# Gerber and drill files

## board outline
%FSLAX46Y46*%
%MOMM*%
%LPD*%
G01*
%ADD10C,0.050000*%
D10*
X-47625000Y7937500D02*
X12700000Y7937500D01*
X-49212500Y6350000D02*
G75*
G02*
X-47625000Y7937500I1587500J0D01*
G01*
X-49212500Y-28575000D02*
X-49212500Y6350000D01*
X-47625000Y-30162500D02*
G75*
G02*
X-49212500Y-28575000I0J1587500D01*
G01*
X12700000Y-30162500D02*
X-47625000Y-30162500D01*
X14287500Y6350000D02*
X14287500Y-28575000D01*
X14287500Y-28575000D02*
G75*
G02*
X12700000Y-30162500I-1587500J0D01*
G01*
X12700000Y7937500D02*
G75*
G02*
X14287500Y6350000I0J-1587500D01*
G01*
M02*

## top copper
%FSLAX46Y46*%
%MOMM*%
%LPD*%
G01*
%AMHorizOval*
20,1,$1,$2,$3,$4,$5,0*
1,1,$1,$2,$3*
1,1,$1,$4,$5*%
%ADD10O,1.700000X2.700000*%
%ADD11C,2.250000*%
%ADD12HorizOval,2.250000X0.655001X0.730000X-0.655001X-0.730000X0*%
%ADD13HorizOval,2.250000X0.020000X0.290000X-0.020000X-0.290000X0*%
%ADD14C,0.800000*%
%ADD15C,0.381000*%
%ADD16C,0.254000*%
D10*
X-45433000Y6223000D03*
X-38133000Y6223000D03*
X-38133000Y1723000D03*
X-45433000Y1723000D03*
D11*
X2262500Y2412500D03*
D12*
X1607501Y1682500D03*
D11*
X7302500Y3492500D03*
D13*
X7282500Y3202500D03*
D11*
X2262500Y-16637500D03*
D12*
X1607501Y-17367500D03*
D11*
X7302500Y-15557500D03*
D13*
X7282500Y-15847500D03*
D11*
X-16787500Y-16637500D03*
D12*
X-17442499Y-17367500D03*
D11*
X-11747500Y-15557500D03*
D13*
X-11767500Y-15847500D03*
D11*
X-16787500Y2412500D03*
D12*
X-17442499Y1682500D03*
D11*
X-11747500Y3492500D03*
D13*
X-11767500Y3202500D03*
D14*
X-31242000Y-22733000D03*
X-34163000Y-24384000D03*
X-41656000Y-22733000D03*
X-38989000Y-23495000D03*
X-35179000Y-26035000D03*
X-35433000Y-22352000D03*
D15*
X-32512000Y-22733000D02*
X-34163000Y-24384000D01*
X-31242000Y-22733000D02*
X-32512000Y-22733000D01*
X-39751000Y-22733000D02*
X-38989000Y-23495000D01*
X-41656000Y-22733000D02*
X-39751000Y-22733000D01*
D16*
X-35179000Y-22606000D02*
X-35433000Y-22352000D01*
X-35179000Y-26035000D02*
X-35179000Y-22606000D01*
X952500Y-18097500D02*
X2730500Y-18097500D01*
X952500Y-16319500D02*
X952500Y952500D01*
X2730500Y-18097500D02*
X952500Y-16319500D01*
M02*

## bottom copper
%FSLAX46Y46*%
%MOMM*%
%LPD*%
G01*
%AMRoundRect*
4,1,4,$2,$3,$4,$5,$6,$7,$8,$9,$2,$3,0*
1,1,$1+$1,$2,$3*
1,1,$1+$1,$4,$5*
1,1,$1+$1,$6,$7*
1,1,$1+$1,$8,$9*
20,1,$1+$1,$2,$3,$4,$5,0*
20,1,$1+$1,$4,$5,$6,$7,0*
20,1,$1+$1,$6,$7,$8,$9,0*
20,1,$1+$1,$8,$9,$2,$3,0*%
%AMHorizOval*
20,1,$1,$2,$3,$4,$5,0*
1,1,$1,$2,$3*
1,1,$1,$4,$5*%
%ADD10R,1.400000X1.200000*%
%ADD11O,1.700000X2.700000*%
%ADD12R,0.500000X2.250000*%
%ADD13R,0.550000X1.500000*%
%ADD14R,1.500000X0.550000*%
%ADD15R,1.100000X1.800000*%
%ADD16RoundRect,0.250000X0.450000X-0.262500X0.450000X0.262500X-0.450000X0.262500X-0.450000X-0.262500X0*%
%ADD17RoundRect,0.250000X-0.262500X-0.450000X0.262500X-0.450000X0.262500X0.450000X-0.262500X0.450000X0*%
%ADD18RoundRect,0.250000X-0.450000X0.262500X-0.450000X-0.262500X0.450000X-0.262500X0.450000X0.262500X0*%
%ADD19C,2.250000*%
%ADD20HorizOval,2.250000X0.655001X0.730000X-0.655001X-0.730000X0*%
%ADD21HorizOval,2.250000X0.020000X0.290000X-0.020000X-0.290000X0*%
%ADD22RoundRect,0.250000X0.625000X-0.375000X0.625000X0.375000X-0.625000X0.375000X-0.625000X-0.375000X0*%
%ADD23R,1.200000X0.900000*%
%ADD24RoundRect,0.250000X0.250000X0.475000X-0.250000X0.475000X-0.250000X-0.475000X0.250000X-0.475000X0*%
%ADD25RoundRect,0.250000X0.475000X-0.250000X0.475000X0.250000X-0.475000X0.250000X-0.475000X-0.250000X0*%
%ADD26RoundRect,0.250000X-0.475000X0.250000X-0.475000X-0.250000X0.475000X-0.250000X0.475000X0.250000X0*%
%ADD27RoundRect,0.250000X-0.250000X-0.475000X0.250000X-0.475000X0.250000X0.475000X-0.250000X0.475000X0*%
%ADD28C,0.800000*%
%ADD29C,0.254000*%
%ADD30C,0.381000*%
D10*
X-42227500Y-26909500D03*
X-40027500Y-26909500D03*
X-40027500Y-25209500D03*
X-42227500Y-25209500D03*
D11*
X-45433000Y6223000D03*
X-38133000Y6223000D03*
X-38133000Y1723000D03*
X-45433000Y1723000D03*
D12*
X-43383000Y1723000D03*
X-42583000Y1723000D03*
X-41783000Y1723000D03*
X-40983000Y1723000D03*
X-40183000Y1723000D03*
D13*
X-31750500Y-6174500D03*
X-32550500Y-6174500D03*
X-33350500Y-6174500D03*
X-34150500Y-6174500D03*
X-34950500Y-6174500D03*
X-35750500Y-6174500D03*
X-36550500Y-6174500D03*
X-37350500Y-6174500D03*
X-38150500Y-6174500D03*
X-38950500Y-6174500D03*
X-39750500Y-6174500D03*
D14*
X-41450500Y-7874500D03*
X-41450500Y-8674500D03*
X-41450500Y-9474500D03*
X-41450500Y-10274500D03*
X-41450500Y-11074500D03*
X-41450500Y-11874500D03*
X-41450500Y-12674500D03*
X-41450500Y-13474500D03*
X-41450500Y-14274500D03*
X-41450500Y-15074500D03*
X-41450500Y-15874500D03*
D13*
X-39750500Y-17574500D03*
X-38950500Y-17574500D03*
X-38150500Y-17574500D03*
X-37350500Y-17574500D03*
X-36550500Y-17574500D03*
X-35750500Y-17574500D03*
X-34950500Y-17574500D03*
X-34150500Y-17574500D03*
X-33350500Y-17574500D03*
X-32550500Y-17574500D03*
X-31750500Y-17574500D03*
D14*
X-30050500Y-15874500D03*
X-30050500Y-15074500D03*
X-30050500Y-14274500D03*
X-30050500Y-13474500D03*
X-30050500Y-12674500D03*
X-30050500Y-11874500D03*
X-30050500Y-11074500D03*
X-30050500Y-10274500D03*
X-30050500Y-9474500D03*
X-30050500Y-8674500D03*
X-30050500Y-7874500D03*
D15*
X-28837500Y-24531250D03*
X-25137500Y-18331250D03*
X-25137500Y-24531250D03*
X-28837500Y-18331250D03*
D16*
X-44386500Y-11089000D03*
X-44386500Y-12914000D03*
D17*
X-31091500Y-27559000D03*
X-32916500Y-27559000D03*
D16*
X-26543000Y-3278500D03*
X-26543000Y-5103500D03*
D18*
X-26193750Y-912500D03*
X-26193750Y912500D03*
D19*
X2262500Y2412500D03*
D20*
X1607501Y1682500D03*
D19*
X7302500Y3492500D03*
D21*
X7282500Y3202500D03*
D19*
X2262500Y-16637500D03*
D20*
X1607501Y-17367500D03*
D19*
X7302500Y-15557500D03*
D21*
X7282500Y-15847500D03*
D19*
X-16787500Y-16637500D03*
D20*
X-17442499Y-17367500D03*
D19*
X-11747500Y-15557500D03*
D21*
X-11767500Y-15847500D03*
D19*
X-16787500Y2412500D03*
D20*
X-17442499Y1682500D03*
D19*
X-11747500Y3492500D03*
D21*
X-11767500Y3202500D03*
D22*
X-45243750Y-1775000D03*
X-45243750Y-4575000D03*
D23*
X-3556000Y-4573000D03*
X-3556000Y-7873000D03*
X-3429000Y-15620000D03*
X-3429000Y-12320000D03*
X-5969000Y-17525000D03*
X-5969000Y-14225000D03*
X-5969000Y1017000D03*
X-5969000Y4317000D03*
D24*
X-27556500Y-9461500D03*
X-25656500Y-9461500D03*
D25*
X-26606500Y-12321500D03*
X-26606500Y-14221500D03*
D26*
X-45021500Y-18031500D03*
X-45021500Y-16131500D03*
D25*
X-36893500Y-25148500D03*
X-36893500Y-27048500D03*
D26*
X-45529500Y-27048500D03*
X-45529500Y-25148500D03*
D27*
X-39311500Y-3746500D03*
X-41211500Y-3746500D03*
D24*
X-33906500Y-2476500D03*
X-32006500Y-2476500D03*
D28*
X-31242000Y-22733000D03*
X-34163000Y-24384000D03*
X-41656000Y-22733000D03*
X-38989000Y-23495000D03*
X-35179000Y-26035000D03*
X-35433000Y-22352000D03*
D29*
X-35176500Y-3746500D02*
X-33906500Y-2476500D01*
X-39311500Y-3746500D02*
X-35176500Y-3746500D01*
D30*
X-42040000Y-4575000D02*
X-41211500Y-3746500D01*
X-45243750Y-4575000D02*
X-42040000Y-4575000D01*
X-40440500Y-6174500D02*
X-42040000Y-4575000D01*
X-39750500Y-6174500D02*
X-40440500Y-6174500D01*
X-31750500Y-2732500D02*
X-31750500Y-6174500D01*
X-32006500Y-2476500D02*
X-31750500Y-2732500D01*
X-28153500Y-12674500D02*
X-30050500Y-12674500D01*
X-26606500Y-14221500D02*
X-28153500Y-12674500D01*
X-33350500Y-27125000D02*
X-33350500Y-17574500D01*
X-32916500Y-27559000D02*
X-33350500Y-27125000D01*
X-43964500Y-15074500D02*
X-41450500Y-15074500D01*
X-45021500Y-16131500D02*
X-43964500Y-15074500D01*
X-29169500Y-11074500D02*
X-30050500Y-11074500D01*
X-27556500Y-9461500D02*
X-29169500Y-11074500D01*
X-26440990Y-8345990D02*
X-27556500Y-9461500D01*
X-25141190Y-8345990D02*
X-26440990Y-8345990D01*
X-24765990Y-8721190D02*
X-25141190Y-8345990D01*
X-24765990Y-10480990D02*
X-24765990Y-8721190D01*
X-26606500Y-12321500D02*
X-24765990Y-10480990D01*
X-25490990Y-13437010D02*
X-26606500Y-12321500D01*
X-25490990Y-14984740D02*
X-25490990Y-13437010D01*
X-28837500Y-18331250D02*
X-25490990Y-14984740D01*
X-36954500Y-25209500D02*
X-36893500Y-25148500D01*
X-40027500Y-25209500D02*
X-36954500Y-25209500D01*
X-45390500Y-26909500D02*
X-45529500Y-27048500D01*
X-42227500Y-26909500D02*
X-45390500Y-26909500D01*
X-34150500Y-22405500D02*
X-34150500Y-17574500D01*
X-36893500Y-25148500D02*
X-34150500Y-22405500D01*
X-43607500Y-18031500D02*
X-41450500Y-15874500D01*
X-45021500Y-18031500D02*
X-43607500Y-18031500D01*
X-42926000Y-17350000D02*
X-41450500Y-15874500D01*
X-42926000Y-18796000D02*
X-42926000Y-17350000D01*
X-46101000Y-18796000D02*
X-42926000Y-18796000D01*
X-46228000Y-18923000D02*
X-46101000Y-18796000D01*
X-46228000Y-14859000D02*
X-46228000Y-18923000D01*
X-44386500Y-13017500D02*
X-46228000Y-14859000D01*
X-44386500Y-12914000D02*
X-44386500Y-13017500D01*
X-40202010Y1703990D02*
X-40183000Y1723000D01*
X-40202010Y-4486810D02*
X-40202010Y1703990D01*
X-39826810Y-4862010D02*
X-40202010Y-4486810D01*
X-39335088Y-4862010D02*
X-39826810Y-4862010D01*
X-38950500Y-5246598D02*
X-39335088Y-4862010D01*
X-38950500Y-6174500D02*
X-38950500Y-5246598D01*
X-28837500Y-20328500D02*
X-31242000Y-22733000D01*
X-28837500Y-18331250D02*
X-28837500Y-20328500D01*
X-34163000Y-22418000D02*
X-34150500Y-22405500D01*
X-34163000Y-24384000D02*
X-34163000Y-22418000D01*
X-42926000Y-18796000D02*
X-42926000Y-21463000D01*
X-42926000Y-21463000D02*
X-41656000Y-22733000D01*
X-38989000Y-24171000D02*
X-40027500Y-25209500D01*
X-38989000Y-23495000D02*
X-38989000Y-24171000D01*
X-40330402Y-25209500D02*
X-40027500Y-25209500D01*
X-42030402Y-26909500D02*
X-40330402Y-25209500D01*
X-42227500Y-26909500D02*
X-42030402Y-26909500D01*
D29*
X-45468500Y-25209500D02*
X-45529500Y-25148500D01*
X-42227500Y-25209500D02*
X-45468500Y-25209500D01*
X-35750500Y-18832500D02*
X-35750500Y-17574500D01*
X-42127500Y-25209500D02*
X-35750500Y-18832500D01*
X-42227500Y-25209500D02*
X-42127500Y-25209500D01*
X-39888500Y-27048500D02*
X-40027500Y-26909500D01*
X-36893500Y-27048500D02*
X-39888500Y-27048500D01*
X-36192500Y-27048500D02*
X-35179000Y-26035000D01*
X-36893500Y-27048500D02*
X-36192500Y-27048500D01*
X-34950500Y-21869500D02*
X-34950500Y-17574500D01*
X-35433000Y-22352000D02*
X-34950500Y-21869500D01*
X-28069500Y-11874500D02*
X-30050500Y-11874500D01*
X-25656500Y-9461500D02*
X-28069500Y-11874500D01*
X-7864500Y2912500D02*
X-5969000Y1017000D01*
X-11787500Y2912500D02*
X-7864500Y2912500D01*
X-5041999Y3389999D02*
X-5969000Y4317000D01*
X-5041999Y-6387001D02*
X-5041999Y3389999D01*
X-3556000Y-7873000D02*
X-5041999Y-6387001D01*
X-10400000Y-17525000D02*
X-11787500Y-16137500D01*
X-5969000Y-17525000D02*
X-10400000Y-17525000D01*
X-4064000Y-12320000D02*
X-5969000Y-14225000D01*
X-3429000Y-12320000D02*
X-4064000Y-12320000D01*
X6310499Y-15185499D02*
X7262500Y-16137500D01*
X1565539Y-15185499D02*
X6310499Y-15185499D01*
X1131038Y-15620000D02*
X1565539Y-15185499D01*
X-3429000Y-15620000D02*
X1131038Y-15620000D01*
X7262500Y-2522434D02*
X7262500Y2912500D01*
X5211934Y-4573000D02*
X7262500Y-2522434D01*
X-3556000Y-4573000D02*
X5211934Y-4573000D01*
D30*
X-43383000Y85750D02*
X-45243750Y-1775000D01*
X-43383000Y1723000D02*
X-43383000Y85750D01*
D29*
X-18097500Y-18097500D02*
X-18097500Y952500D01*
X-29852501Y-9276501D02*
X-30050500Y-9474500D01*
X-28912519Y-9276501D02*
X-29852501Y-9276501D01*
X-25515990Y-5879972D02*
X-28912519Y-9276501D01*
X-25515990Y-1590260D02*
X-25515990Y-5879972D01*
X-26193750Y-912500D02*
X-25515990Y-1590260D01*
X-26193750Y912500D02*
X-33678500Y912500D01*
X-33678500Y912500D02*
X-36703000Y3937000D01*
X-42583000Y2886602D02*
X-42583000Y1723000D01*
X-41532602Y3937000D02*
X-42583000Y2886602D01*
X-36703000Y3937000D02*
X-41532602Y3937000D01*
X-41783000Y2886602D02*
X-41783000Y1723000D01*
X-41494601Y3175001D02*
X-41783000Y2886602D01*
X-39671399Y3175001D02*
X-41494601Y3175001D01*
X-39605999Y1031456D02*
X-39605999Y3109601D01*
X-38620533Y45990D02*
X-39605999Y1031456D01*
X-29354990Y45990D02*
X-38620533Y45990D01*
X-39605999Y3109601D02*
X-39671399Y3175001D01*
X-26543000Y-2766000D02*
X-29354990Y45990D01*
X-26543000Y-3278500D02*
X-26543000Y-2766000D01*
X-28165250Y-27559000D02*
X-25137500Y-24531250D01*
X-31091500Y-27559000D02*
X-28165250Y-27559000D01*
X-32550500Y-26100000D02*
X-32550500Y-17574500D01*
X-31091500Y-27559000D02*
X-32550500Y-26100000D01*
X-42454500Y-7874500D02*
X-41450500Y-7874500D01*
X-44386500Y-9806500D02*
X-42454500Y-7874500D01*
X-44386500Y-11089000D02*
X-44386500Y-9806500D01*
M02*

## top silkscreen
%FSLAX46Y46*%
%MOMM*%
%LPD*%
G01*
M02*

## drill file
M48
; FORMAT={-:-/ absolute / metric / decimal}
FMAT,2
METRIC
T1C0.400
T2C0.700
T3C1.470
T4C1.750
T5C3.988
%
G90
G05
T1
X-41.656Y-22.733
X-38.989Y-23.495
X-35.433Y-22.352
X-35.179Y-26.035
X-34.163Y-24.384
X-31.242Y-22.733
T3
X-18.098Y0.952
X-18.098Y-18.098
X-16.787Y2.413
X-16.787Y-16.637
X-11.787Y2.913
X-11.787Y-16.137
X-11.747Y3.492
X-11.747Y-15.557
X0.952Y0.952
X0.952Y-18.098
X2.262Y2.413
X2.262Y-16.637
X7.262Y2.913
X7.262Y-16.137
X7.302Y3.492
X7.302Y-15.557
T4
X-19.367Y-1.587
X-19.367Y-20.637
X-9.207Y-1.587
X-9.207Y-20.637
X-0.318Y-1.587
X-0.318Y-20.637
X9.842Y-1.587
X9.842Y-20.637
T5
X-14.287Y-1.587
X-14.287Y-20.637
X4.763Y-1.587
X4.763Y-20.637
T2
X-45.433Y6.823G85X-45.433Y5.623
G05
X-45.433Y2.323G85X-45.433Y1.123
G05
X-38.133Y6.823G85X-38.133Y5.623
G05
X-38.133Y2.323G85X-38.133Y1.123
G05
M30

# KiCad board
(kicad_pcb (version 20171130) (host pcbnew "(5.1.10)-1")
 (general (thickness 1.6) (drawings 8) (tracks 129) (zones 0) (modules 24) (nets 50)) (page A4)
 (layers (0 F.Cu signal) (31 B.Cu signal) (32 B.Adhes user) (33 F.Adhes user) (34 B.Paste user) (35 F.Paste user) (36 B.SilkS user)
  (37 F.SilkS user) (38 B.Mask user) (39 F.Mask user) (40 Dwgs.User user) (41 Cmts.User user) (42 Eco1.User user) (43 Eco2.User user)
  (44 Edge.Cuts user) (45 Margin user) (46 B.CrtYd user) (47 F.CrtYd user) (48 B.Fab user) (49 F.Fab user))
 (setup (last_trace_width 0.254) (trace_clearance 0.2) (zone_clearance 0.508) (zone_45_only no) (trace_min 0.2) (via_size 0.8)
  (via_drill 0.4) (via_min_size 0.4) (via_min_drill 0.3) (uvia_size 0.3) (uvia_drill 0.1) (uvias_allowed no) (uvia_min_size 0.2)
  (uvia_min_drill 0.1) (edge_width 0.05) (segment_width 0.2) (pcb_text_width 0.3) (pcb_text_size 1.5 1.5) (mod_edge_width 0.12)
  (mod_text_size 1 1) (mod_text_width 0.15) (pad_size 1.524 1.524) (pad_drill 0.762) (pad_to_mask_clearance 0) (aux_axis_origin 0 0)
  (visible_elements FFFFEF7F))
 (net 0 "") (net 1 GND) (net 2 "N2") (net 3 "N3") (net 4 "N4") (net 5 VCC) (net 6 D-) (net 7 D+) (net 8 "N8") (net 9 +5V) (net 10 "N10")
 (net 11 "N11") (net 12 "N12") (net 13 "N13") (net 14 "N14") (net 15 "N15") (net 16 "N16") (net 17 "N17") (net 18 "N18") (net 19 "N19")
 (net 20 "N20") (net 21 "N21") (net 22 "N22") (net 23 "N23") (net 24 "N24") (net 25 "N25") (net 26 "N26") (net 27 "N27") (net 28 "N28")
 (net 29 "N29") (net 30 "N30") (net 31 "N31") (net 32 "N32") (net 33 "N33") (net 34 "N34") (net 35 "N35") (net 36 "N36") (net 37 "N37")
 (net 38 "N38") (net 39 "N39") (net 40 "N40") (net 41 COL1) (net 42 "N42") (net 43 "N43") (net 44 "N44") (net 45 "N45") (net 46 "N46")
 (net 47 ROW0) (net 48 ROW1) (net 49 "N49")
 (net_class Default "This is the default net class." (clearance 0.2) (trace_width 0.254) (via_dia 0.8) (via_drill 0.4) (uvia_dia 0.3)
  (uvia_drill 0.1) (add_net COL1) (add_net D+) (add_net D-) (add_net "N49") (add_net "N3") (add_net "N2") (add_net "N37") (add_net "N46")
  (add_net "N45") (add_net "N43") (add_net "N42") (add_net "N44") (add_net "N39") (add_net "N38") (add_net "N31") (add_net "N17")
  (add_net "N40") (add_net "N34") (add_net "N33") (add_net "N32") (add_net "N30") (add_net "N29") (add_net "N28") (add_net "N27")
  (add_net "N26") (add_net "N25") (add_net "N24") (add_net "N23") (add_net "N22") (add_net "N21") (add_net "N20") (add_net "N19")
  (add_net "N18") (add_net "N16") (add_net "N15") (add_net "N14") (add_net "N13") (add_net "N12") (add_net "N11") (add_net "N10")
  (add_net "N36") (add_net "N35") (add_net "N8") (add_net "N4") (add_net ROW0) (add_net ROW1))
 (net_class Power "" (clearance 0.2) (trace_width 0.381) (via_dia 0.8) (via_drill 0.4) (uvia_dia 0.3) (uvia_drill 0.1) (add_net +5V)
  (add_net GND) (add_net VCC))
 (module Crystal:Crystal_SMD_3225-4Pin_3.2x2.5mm (layer B.Cu) (at -41.1275 26.0595)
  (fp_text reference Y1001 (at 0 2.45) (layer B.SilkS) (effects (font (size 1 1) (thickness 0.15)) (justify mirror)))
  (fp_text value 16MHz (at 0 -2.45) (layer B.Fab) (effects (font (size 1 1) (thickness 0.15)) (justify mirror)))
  (pad 4 smd rect (at -1.1 0.85) (size 1.4 1.2) (layers B.Cu B.Paste B.Mask) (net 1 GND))
  (pad 3 smd rect (at 1.1 0.85) (size 1.4 1.2) (layers B.Cu B.Paste B.Mask) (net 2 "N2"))
  (pad 2 smd rect (at 1.1 -0.85) (size 1.4 1.2) (layers B.Cu B.Paste B.Mask) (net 1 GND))
  (pad 1 smd rect (at -1.1 -0.85) (size 1.4 1.2) (layers B.Cu B.Paste B.Mask) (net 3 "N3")))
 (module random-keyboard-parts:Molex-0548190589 (layer B.Cu) (at -41.783 -6.223 270)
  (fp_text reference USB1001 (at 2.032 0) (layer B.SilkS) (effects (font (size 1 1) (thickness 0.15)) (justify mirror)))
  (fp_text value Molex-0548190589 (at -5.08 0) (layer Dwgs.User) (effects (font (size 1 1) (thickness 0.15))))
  (pad 6 thru_hole oval (at 0 3.65 270) (size 2.7 1.7) (drill oval 1.9 0.7) (layers *.Cu *.Mask) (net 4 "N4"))
  (pad 6 thru_hole oval (at 0 -3.65 270) (size 2.7 1.7) (drill oval 1.9 0.7) (layers *.Cu *.Mask) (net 4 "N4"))
  (pad 6 thru_hole oval (at 4.5 -3.65 270) (size 2.7 1.7) (drill oval 1.9 0.7) (layers *.Cu *.Mask) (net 4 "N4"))
  (pad 6 thru_hole oval (at 4.5 3.65 270) (size 2.7 1.7) (drill oval 1.9 0.7) (layers *.Cu *.Mask) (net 4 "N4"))
  (pad 5 smd rect (at 4.5 1.6 270) (size 2.25 0.5) (layers B.Cu B.Paste B.Mask) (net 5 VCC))
  (pad 4 smd rect (at 4.5 0.8 270) (size 2.25 0.5) (layers B.Cu B.Paste B.Mask) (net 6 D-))
  (pad 3 smd rect (at 4.5 0 270) (size 2.25 0.5) (layers B.Cu B.Paste B.Mask) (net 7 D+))
  (pad 2 smd rect (at 4.5 -0.8 270) (size 2.25 0.5) (layers B.Cu B.Paste B.Mask) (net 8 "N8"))
  (pad 1 smd rect (at 4.5 -1.6 270) (size 2.25 0.5) (layers B.Cu B.Paste B.Mask) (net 1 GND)))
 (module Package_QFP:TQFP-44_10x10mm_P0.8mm (layer B.Cu) (at -35.7505 11.8745 180)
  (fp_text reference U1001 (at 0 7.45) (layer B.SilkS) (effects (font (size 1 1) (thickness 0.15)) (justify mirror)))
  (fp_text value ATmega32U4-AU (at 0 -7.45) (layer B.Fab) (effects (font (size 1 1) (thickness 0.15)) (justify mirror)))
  (pad 44 smd rect (at -4 5.7 90) (size 1.5 0.55) (layers B.Cu B.Paste B.Mask) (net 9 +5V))
  (pad 43 smd rect (at -3.2 5.7 90) (size 1.5 0.55) (layers B.Cu B.Paste B.Mask) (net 1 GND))
  (pad 42 smd rect (at -2.4 5.7 90) (size 1.5 0.55) (layers B.Cu B.Paste B.Mask) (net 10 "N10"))
  (pad 41 smd rect (at -1.6 5.7 90) (size 1.5 0.55) (layers B.Cu B.Paste B.Mask) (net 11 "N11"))
  (pad 40 smd rect (at -0.8 5.7 90) (size 1.5 0.55) (layers B.Cu B.Paste B.Mask) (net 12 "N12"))
  (pad 39 smd rect (at 0 5.7 90) (size 1.5 0.55) (layers B.Cu B.Paste B.Mask) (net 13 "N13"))
  (pad 38 smd rect (at 0.8 5.7 90) (size 1.5 0.55) (layers B.Cu B.Paste B.Mask) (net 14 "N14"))
  (pad 37 smd rect (at 1.6 5.7 90) (size 1.5 0.55) (layers B.Cu B.Paste B.Mask) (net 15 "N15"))
  (pad 36 smd rect (at 2.4 5.7 90) (size 1.5 0.55) (layers B.Cu B.Paste B.Mask) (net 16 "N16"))
  (pad 35 smd rect (at 3.2 5.7 90) (size 1.5 0.55) (layers B.Cu B.Paste B.Mask) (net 1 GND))
  (pad 34 smd rect (at 4 5.7 90) (size 1.5 0.55) (layers B.Cu B.Paste B.Mask) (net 9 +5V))
  (pad 33 smd rect (at 5.7 4 180) (size 1.5 0.55) (layers B.Cu B.Paste B.Mask) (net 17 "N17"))
  (pad 32 smd rect (at 5.7 3.2 180) (size 1.5 0.55) (layers B.Cu B.Paste B.Mask) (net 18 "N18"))
  (pad 31 smd rect (at 5.7 2.4 180) (size 1.5 0.55) (layers B.Cu B.Paste B.Mask) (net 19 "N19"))
  (pad 30 smd rect (at 5.7 1.6 180) (size 1.5 0.55) (layers B.Cu B.Paste B.Mask) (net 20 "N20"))
  (pad 29 smd rect (at 5.7 0.8 180) (size 1.5 0.55) (layers B.Cu B.Paste B.Mask) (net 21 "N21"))
  (pad 28 smd rect (at 5.7 0 180) (size 1.5 0.55) (layers B.Cu B.Paste B.Mask) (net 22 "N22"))
  (pad 27 smd rect (at 5.7 -0.8 180) (size 1.5 0.55) (layers B.Cu B.Paste B.Mask) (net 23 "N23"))
  (pad 26 smd rect (at 5.7 -1.6 180) (size 1.5 0.55) (layers B.Cu B.Paste B.Mask) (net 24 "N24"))
  (pad 25 smd rect (at 5.7 -2.4 180) (size 1.5 0.55) (layers B.Cu B.Paste B.Mask) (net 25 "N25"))
  (pad 24 smd rect (at 5.7 -3.2 180) (size 1.5 0.55) (layers B.Cu B.Paste B.Mask) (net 9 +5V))
  (pad 23 smd rect (at 5.7 -4 180) (size 1.5 0.55) (layers B.Cu B.Paste B.Mask) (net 1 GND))
  (pad 22 smd rect (at 4 -5.7 90) (size 1.5 0.55) (layers B.Cu B.Paste B.Mask) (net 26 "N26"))
  (pad 21 smd rect (at 3.2 -5.7 90) (size 1.5 0.55) (layers B.Cu B.Paste B.Mask) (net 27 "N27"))
  (pad 20 smd rect (at 2.4 -5.7 90) (size 1.5 0.55) (layers B.Cu B.Paste B.Mask) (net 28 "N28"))
  (pad 19 smd rect (at 1.6 -5.7 90) (size 1.5 0.55) (layers B.Cu B.Paste B.Mask) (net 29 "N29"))
  (pad 18 smd rect (at 0.8 -5.7 90) (size 1.5 0.55) (layers B.Cu B.Paste B.Mask) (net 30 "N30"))
  (pad 17 smd rect (at 0 -5.7 90) (size 1.5 0.55) (layers B.Cu B.Paste B.Mask) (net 3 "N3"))
  (pad 16 smd rect (at -0.8 -5.7 90) (size 1.5 0.55) (layers B.Cu B.Paste B.Mask) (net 2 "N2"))
  (pad 15 smd rect (at -1.6 -5.7 90) (size 1.5 0.55) (layers B.Cu B.Paste B.Mask) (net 1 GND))
  (pad 14 smd rect (at -2.4 -5.7 90) (size 1.5 0.55) (layers B.Cu B.Paste B.Mask) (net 9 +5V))
  (pad 13 smd rect (at -3.2 -5.7 90) (size 1.5 0.55) (layers B.Cu B.Paste B.Mask) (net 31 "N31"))
  (pad 12 smd rect (at -4 -5.7 90) (size 1.5 0.55) (layers B.Cu B.Paste B.Mask) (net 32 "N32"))
  (pad 11 smd rect (at -5.7 -4 180) (size 1.5 0.55) (layers B.Cu B.Paste B.Mask) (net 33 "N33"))
  (pad 10 smd rect (at -5.7 -3.2 180) (size 1.5 0.55) (layers B.Cu B.Paste B.Mask) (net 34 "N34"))
  (pad 9 smd rect (at -5.7 -2.4 180) (size 1.5 0.55) (layers B.Cu B.Paste B.Mask) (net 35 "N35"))
  (pad 8 smd rect (at -5.7 -1.6 180) (size 1.5 0.55) (layers B.Cu B.Paste B.Mask) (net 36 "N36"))
  (pad 7 smd rect (at -5.7 -0.8 180) (size 1.5 0.55) (layers B.Cu B.Paste B.Mask) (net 9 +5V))
  (pad 6 smd rect (at -5.7 0 180) (size 1.5 0.55) (layers B.Cu B.Paste B.Mask) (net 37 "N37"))
  (pad 5 smd rect (at -5.7 0.8 180) (size 1.5 0.55) (layers B.Cu B.Paste B.Mask) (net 1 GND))
  (pad 4 smd rect (at -5.7 1.6 180) (size 1.5 0.55) (layers B.Cu B.Paste B.Mask) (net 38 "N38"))
  (pad 3 smd rect (at -5.7 2.4 180) (size 1.5 0.55) (layers B.Cu B.Paste B.Mask) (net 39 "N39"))
  (pad 2 smd rect (at -5.7 3.2 180) (size 1.5 0.55) (layers B.Cu B.Paste B.Mask) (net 9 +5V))
  (pad 1 smd rect (at -5.7 4 180) (size 1.5 0.55) (layers B.Cu B.Paste B.Mask) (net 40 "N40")))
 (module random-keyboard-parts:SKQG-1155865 (layer B.Cu) (at -26.9875 21.43125 90)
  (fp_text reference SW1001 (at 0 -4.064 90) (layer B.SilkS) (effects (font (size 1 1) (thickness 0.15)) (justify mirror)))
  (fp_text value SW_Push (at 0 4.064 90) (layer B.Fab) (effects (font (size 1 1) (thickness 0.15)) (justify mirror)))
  (pad 4 smd rect (at -3.1 -1.85 90) (size 1.8 1.1) (layers B.Cu B.Paste B.Mask))
  (pad 3 smd rect (at 3.1 1.85 90) (size 1.8 1.1) (layers B.Cu B.Paste B.Mask))
  (pad 2 smd rect (at -3.1 1.85 90) (size 1.8 1.1) (layers B.Cu B.Paste B.Mask) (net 31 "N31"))
  (pad 1 smd rect (at 3.1 -1.85 90) (size 1.8 1.1) (layers B.Cu B.Paste B.Mask) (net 1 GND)))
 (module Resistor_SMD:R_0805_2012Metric (layer B.Cu) (at -44.3865 12.0015 90)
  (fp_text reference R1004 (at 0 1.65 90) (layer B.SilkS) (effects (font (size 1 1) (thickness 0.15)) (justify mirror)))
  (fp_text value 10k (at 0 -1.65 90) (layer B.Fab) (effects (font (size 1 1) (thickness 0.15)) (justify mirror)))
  (pad 2 smd roundrect (at 0.9125 0 90) (size 1.025 1.4) (layers B.Cu B.Paste B.Mask) (roundrect_rratio 0.243902) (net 17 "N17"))
  (pad 1 smd roundrect (at -0.9125 0 90) (size 1.025 1.4) (layers B.Cu B.Paste B.Mask) (roundrect_rratio 0.243902) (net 1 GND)))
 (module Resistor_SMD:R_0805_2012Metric (layer B.Cu) (at -32.004 27.559)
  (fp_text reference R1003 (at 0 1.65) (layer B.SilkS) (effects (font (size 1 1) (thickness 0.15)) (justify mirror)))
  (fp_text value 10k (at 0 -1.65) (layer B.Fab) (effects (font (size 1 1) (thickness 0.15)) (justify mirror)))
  (pad 2 smd roundrect (at 0.9125 0) (size 1.025 1.4) (layers B.Cu B.Paste B.Mask) (roundrect_rratio 0.243902) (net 31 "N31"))
  (pad 1 smd roundrect (at -0.9125 0) (size 1.025 1.4) (layers B.Cu B.Paste B.Mask) (roundrect_rratio 0.243902) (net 9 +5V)))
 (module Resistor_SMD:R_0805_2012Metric (layer B.Cu) (at -26.543 4.191 90)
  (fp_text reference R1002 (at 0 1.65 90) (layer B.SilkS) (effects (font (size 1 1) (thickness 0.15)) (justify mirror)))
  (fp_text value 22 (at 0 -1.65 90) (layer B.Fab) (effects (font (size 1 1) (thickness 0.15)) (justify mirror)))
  (pad 2 smd roundrect (at 0.9125 0 90) (size 1.025 1.4) (layers B.Cu B.Paste B.Mask) (roundrect_rratio 0.243902) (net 7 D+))
  (pad 1 smd roundrect (at -0.9125 0 90) (size 1.025 1.4) (layers B.Cu B.Paste B.Mask) (roundrect_rratio 0.243902) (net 38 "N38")))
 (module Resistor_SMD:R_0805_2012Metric (layer B.Cu) (at -26.19375 0 270)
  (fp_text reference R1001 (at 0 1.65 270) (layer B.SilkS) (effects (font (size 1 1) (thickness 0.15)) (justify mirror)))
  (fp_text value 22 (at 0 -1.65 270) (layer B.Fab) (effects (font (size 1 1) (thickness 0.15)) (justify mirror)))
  (pad 2 smd roundrect (at 0.9125 0 270) (size 1.025 1.4) (layers B.Cu B.Paste B.Mask) (roundrect_rratio 0.243902) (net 39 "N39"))
  (pad 1 smd roundrect (at -0.9125 0 270) (size 1.025 1.4) (layers B.Cu B.Paste B.Mask) (roundrect_rratio 0.243902) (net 6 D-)))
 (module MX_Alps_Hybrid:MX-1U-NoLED (layer F.Cu) (at 4.7625 1.5875)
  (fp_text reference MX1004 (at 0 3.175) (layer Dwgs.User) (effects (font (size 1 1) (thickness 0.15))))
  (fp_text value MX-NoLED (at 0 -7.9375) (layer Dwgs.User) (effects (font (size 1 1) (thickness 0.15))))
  (pad "" np_thru_hole circle (at 5.08 0 48.0996) (size 1.75 1.75) (drill 1.75) (layers *.Cu *.Mask))
  (pad "" np_thru_hole circle (at -5.08 0 48.0996) (size 1.75 1.75) (drill 1.75) (layers *.Cu *.Mask))
  (pad 1 thru_hole circle (at -2.5 -4) (size 2.25 2.25) (drill 1.47) (layers *.Cu B.Mask) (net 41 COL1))
  (pad "" np_thru_hole circle (at 0 0) (size 3.9878 3.9878) (drill 3.9878) (layers *.Cu *.Mask))
  (pad 1 thru_hole oval (at -3.81 -2.54 48.0996) (size 4.211556 2.25) (drill 1.47 (offset 0.980778 0)) (layers *.Cu B.Mask) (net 41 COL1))
  (pad 2 thru_hole circle (at 2.54 -5.08) (size 2.25 2.25) (drill 1.47) (layers *.Cu B.Mask) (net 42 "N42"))
  (pad 2 thru_hole oval (at 2.5 -4.5 86.0548) (size 2.831378 2.25) (drill 1.47 (offset 0.290689 0)) (layers *.Cu B.Mask) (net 42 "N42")))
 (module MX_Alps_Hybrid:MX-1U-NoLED (layer F.Cu) (at 4.7625 20.6375)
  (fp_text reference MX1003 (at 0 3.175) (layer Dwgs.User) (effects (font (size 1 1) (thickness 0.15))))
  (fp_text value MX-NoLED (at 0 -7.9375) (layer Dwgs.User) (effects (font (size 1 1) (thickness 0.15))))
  (pad "" np_thru_hole circle (at 5.08 0 48.0996) (size 1.75 1.75) (drill 1.75) (layers *.Cu *.Mask))
  (pad "" np_thru_hole circle (at -5.08 0 48.0996) (size 1.75 1.75) (drill 1.75) (layers *.Cu *.Mask))
  (pad 1 thru_hole circle (at -2.5 -4) (size 2.25 2.25) (drill 1.47) (layers *.Cu B.Mask) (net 41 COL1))
  (pad "" np_thru_hole circle (at 0 0) (size 3.9878 3.9878) (drill 3.9878) (layers *.Cu *.Mask))
  (pad 1 thru_hole oval (at -3.81 -2.54 48.0996) (size 4.211556 2.25) (drill 1.47 (offset 0.980778 0)) (layers *.Cu B.Mask) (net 41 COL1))
  (pad 2 thru_hole circle (at 2.54 -5.08) (size 2.25 2.25) (drill 1.47) (layers *.Cu B.Mask) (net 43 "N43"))
  (pad 2 thru_hole oval (at 2.5 -4.5 86.0548) (size 2.831378 2.25) (drill 1.47 (offset 0.290689 0)) (layers *.Cu B.Mask) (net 43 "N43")))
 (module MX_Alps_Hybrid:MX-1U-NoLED (layer F.Cu) (at -14.2875 20.6375)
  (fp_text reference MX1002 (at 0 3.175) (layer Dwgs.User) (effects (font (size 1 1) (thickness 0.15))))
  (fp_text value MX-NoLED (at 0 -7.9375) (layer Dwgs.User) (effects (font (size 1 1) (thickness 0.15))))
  (pad "" np_thru_hole circle (at 5.08 0 48.0996) (size 1.75 1.75) (drill 1.75) (layers *.Cu *.Mask))
  (pad "" np_thru_hole circle (at -5.08 0 48.0996) (size 1.75 1.75) (drill 1.75) (layers *.Cu *.Mask))
  (pad 1 thru_hole circle (at -2.5 -4) (size 2.25 2.25) (drill 1.47) (layers *.Cu B.Mask) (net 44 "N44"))
  (pad "" np_thru_hole circle (at 0 0) (size 3.9878 3.9878) (drill 3.9878) (layers *.Cu *.Mask))
  (pad 1 thru_hole oval (at -3.81 -2.54 48.0996) (size 4.211556 2.25) (drill 1.47 (offset 0.980778 0)) (layers *.Cu B.Mask) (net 44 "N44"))
  (pad 2 thru_hole circle (at 2.54 -5.08) (size 2.25 2.25) (drill 1.47) (layers *.Cu B.Mask) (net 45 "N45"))
  (pad 2 thru_hole oval (at 2.5 -4.5 86.0548) (size 2.831378 2.25) (drill 1.47 (offset 0.290689 0)) (layers *.Cu B.Mask) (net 45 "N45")))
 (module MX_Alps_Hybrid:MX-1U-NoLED (layer F.Cu) (at -14.2875 1.5875)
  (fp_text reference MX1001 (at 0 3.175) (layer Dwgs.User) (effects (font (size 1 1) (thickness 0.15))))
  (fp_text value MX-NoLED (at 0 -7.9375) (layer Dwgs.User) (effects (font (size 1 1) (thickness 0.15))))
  (pad "" np_thru_hole circle (at 5.08 0 48.0996) (size 1.75 1.75) (drill 1.75) (layers *.Cu *.Mask))
  (pad "" np_thru_hole circle (at -5.08 0 48.0996) (size 1.75 1.75) (drill 1.75) (layers *.Cu *.Mask))
  (pad 1 thru_hole circle (at -2.5 -4) (size 2.25 2.25) (drill 1.47) (layers *.Cu B.Mask) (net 44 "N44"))
  (pad "" np_thru_hole circle (at 0 0) (size 3.9878 3.9878) (drill 3.9878) (layers *.Cu *.Mask))
  (pad 1 thru_hole oval (at -3.81 -2.54 48.0996) (size 4.211556 2.25) (drill 1.47 (offset 0.980778 0)) (layers *.Cu B.Mask) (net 44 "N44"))
  (pad 2 thru_hole circle (at 2.54 -5.08) (size 2.25 2.25) (drill 1.47) (layers *.Cu B.Mask) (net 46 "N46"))
  (pad 2 thru_hole oval (at 2.5 -4.5 86.0548) (size 2.831378 2.25) (drill 1.47 (offset 0.290689 0)) (layers *.Cu B.Mask) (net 46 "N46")))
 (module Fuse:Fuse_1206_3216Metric (layer B.Cu) (at -45.24375 3.175 90)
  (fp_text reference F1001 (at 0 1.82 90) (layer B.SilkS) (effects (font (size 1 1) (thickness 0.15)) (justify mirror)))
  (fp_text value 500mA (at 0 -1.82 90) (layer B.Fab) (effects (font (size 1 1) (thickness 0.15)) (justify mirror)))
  (pad 2 smd roundrect (at 1.4 0 90) (size 1.25 1.75) (layers B.Cu B.Paste B.Mask) (roundrect_rratio 0.2) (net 5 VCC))
  (pad 1 smd roundrect (at -1.4 0 90) (size 1.25 1.75) (layers B.Cu B.Paste B.Mask) (roundrect_rratio 0.2) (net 9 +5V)))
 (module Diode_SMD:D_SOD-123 (layer B.Cu) (at -3.556 6.223 90)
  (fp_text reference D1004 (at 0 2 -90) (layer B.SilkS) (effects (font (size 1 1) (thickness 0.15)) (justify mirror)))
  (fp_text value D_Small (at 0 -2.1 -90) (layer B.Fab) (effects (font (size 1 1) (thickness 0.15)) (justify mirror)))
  (pad 2 smd rect (at 1.65 0 90) (size 0.9 1.2) (layers B.Cu B.Paste B.Mask) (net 42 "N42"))
  (pad 1 smd rect (at -1.65 0 90) (size 0.9 1.2) (layers B.Cu B.Paste B.Mask) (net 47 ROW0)))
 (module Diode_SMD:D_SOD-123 (layer B.Cu) (at -3.429 13.97 270)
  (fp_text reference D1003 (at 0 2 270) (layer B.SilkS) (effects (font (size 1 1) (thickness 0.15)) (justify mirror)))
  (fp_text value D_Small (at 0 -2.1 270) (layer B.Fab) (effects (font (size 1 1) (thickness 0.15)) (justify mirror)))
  (pad 2 smd rect (at 1.65 0 270) (size 0.9 1.2) (layers B.Cu B.Paste B.Mask) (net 43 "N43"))
  (pad 1 smd rect (at -1.65 0 270) (size 0.9 1.2) (layers B.Cu B.Paste B.Mask) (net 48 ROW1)))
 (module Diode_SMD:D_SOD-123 (layer B.Cu) (at -5.969 15.875 270)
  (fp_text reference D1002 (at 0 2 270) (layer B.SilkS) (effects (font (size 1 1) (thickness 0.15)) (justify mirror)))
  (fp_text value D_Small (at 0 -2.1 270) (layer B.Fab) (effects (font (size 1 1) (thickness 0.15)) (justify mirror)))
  (pad 2 smd rect (at 1.65 0 270) (size 0.9 1.2) (layers B.Cu B.Paste B.Mask) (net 45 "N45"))
  (pad 1 smd rect (at -1.65 0 270) (size 0.9 1.2) (layers B.Cu B.Paste B.Mask) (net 48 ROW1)))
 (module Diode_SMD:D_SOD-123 (layer B.Cu) (at -5.969 -2.667 270)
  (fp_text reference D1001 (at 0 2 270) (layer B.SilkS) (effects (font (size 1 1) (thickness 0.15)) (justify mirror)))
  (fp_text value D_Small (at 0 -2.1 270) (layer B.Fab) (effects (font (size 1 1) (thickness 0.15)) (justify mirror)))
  (pad 2 smd rect (at 1.65 0 270) (size 0.9 1.2) (layers B.Cu B.Paste B.Mask) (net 46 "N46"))
  (pad 1 smd rect (at -1.65 0 270) (size 0.9 1.2) (layers B.Cu B.Paste B.Mask) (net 47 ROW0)))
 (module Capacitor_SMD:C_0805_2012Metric (layer B.Cu) (at -26.6065 9.4615 180)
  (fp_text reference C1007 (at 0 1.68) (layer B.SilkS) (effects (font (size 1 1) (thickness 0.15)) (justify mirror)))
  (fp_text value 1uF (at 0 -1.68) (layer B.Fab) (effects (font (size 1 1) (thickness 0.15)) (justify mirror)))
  (pad 2 smd roundrect (at 0.95 0 180) (size 1 1.45) (layers B.Cu B.Paste B.Mask) (roundrect_rratio 0.25) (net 1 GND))
  (pad 1 smd roundrect (at -0.95 0 180) (size 1 1.45) (layers B.Cu B.Paste B.Mask) (roundrect_rratio 0.25) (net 37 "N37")))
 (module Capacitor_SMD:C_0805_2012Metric (layer B.Cu) (at -26.6065 13.2715 90)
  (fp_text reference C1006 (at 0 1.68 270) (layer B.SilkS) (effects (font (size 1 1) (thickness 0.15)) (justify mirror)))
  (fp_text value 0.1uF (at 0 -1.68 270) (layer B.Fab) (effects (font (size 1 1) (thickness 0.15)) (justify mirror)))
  (pad 2 smd roundrect (at 0.95 0 90) (size 1 1.45) (layers B.Cu B.Paste B.Mask) (roundrect_rratio 0.25) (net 1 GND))
  (pad 1 smd roundrect (at -0.95 0 90) (size 1 1.45) (layers B.Cu B.Paste B.Mask) (roundrect_rratio 0.25) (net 9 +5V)))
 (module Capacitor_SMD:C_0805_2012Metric (layer B.Cu) (at -45.0215 17.0815 270)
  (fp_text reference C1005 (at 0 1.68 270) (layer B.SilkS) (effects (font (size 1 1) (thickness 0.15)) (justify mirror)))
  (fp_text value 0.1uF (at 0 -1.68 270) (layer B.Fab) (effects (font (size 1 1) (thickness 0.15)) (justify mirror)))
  (pad 2 smd roundrect (at 0.95 0 270) (size 1 1.45) (layers B.Cu B.Paste B.Mask) (roundrect_rratio 0.25) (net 1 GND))
  (pad 1 smd roundrect (at -0.95 0 270) (size 1 1.45) (layers B.Cu B.Paste B.Mask) (roundrect_rratio 0.25) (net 9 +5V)))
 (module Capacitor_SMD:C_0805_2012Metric (layer B.Cu) (at -36.8935 26.0985 90)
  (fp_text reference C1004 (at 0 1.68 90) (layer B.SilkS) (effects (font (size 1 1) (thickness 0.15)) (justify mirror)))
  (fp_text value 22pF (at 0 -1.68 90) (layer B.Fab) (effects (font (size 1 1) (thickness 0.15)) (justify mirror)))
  (pad 2 smd roundrect (at 0.95 0 90) (size 1 1.45) (layers B.Cu B.Paste B.Mask) (roundrect_rratio 0.25) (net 1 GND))
  (pad 1 smd roundrect (at -0.95 0 90) (size 1 1.45) (layers B.Cu B.Paste B.Mask) (roundrect_rratio 0.25) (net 2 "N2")))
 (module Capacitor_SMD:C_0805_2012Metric (layer B.Cu) (at -45.5295 26.0985 270)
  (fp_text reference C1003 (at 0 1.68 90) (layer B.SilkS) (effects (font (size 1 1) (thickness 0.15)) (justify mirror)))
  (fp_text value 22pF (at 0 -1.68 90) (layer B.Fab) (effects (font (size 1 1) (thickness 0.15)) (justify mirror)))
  (pad 2 smd roundrect (at 0.95 0 270) (size 1 1.45) (layers B.Cu B.Paste B.Mask) (roundrect_rratio 0.25) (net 1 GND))
  (pad 1 smd roundrect (at -0.95 0 270) (size 1 1.45) (layers B.Cu B.Paste B.Mask) (roundrect_rratio 0.25) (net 3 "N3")))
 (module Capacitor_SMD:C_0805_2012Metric (layer B.Cu) (at -40.2615 3.7465)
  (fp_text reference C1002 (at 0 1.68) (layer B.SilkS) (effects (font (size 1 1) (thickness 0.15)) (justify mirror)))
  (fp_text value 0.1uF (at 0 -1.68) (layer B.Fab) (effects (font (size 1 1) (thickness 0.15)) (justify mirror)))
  (pad 2 smd roundrect (at 0.95 0) (size 1 1.45) (layers B.Cu B.Paste B.Mask) (roundrect_rratio 0.25) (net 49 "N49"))
  (pad 1 smd roundrect (at -0.95 0) (size 1 1.45) (layers B.Cu B.Paste B.Mask) (roundrect_rratio 0.25) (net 9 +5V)))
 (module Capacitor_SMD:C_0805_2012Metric (layer B.Cu) (at -32.9565 2.4765 180)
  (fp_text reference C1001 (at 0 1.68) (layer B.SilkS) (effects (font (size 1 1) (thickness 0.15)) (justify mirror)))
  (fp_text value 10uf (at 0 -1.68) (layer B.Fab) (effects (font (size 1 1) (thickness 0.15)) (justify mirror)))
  (pad 2 smd roundrect (at 0.95 0 180) (size 1 1.45) (layers B.Cu B.Paste B.Mask) (roundrect_rratio 0.25) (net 49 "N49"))
  (pad 1 smd roundrect (at -0.95 0 180) (size 1 1.45) (layers B.Cu B.Paste B.Mask) (roundrect_rratio 0.25) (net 9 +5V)))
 (gr_line (start -47.625 -7.9375) (end 12.7 -7.9375) (layer Edge.Cuts) (width 0.05))
 (gr_arc (start -47.625 -6.35) (end -47.625 -7.9375) (angle -90) (layer Edge.Cuts) (width 0.05))
 (gr_line (start -49.2125 28.575) (end -49.2125 -6.35) (layer Edge.Cuts) (width 0.05))
 (gr_arc (start -47.625 28.575) (end -49.2125 28.575) (angle -90) (layer Edge.Cuts) (width 0.05))
 (gr_line (start 12.7 30.1625) (end -47.625 30.1625) (layer Edge.Cuts) (width 0.05))
 (gr_line (start 14.2875 -6.35) (end 14.2875 28.575) (layer Edge.Cuts) (width 0.05))
 (gr_arc (start 12.7 28.575) (end 12.7 30.1625) (angle -90) (layer Edge.Cuts) (width 0.05))
 (gr_arc (start 12.7 -6.35) (end 14.2875 -6.35) (angle -90) (layer Edge.Cuts) (width 0.05))
 (segment (start -35.1765 3.7465) (end -33.9065 2.4765) (width 0.254) (layer B.Cu) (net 49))
 (segment (start -39.3115 3.7465) (end -35.1765 3.7465) (width 0.254) (layer B.Cu) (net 49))
 (segment (start -42.04 4.575) (end -41.2115 3.7465) (width 0.381) (layer B.Cu) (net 9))
 (segment (start -45.24375 4.575) (end -42.04 4.575) (width 0.381) (layer B.Cu) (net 9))
 (segment (start -40.4405 6.1745) (end -42.04 4.575) (width 0.381) (layer B.Cu) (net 9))
 (segment (start -39.7505 6.1745) (end -40.4405 6.1745) (width 0.381) (layer B.Cu) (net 9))
 (segment (start -31.7505 2.7325) (end -31.7505 6.1745) (width 0.381) (layer B.Cu) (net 9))
 (segment (start -32.0065 2.4765) (end -31.7505 2.7325) (width 0.381) (layer B.Cu) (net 9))
 (segment (start -28.1535 12.6745) (end -30.0505 12.6745) (width 0.381) (layer B.Cu) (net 9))
 (segment (start -26.6065 14.2215) (end -28.1535 12.6745) (width 0.381) (layer B.Cu) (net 9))
 (segment (start -33.3505 27.125) (end -33.3505 17.5745) (width 0.381) (layer B.Cu) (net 9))
 (segment (start -32.9165 27.559) (end -33.3505 27.125) (width 0.381) (layer B.Cu) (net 9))
 (segment (start -43.9645 15.0745) (end -41.4505 15.0745) (width 0.381) (layer B.Cu) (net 9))
 (segment (start -45.0215 16.1315) (end -43.9645 15.0745) (width 0.381) (layer B.Cu) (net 9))
 (segment (start -29.1695 11.0745) (end -30.0505 11.0745) (width 0.381) (layer B.Cu) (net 1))
 (segment (start -27.5565 9.4615) (end -29.1695 11.0745) (width 0.381) (layer B.Cu) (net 1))
 (segment (start -26.44099 8.34599) (end -27.5565 9.4615) (width 0.381) (layer B.Cu) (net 1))
 (segment (start -25.14119 8.34599) (end -26.44099 8.34599) (width 0.381) (layer B.Cu) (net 1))
 (segment (start -24.76599 8.72119) (end -25.14119 8.34599) (width 0.381) (layer B.Cu) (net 1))
 (segment (start -24.76599 10.48099) (end -24.76599 8.72119) (width 0.381) (layer B.Cu) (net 1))
 (segment (start -26.6065 12.3215) (end -24.76599 10.48099) (width 0.381) (layer B.Cu) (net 1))
 (segment (start -25.49099 13.43701) (end -26.6065 12.3215) (width 0.381) (layer B.Cu) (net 1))
 (segment (start -25.49099 14.98474) (end -25.49099 13.43701) (width 0.381) (layer B.Cu) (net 1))
 (segment (start -28.8375 18.33125) (end -25.49099 14.98474) (width 0.381) (layer B.Cu) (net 1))
 (segment (start -36.9545 25.2095) (end -36.8935 25.1485) (width 0.381) (layer B.Cu) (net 1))
 (segment (start -40.0275 25.2095) (end -36.9545 25.2095) (width 0.381) (layer B.Cu) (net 1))
 (segment (start -45.3905 26.9095) (end -45.5295 27.0485) (width 0.381) (layer B.Cu) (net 1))
 (segment (start -42.2275 26.9095) (end -45.3905 26.9095) (width 0.381) (layer B.Cu) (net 1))
 (segment (start -34.1505 22.4055) (end -34.1505 17.5745) (width 0.381) (layer B.Cu) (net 1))
 (segment (start -36.8935 25.1485) (end -34.1505 22.4055) (width 0.381) (layer B.Cu) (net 1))
 (segment (start -43.6075 18.0315) (end -41.4505 15.8745) (width 0.381) (layer B.Cu) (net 1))
 (segment (start -45.0215 18.0315) (end -43.6075 18.0315) (width 0.381) (layer B.Cu) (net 1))
 (segment (start -42.926 17.35) (end -41.4505 15.8745) (width 0.381) (layer B.Cu) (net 1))
 (segment (start -42.926 18.796) (end -42.926 17.35) (width 0.381) (layer B.Cu) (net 1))
 (segment (start -46.101 18.796) (end -42.926 18.796) (width 0.381) (layer B.Cu) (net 1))
 (segment (start -46.228 18.923) (end -46.101 18.796) (width 0.381) (layer B.Cu) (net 1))
 (segment (start -46.228 14.859) (end -46.228 18.923) (width 0.381) (layer B.Cu) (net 1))
 (segment (start -44.3865 13.0175) (end -46.228 14.859) (width 0.381) (layer B.Cu) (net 1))
 (segment (start -44.3865 12.914) (end -44.3865 13.0175) (width 0.381) (layer B.Cu) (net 1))
 (segment (start -40.20201 -1.70399) (end -40.183 -1.723) (width 0.381) (layer B.Cu) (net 1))
 (segment (start -40.20201 4.48681) (end -40.20201 -1.70399) (width 0.381) (layer B.Cu) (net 1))
 (segment (start -39.82681 4.86201) (end -40.20201 4.48681) (width 0.381) (layer B.Cu) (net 1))
 (segment (start -39.335088 4.86201) (end -39.82681 4.86201) (width 0.381) (layer B.Cu) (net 1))
 (segment (start -38.9505 5.246598) (end -39.335088 4.86201) (width 0.381) (layer B.Cu) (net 1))
 (segment (start -38.9505 6.1745) (end -38.9505 5.246598) (width 0.381) (layer B.Cu) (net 1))
 (via (at -31.242 22.733) (size 0.8) (drill 0.4) (layers F.Cu B.Cu) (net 1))
 (segment (start -28.8375 20.3285) (end -31.242 22.733) (width 0.381) (layer B.Cu) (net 1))
 (segment (start -28.8375 18.33125) (end -28.8375 20.3285) (width 0.381) (layer B.Cu) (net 1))
 (via (at -34.163 24.384) (size 0.8) (drill 0.4) (layers F.Cu B.Cu) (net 1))
 (segment (start -32.512 22.733) (end -34.163 24.384) (width 0.381) (layer F.Cu) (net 1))
 (segment (start -31.242 22.733) (end -32.512 22.733) (width 0.381) (layer F.Cu) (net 1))
 (segment (start -34.163 22.418) (end -34.1505 22.4055) (width 0.381) (layer B.Cu) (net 1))
 (segment (start -34.163 24.384) (end -34.163 22.418) (width 0.381) (layer B.Cu) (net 1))
 (segment (start -42.926 18.796) (end -42.926 21.463) (width 0.381) (layer B.Cu) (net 1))
 (via (at -41.656 22.733) (size 0.8) (drill 0.4) (layers F.Cu B.Cu) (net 1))
 (segment (start -42.926 21.463) (end -41.656 22.733) (width 0.381) (layer B.Cu) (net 1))
 (via (at -38.989 23.495) (size 0.8) (drill 0.4) (layers F.Cu B.Cu) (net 1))
 (segment (start -39.751 22.733) (end -38.989 23.495) (width 0.381) (layer F.Cu) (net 1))
 (segment (start -41.656 22.733) (end -39.751 22.733) (width 0.381) (layer F.Cu) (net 1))
 (segment (start -38.989 24.171) (end -40.0275 25.2095) (width 0.381) (layer B.Cu) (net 1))
 (segment (start -38.989 23.495) (end -38.989 24.171) (width 0.381) (layer B.Cu) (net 1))
 (segment (start -40.330402 25.2095) (end -40.0275 25.2095) (width 0.381) (layer B.Cu) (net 1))
 (segment (start -42.030402 26.9095) (end -40.330402 25.2095) (width 0.381) (layer B.Cu) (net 1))
 (segment (start -42.2275 26.9095) (end -42.030402 26.9095) (width 0.381) (layer B.Cu) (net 1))
 (segment (start -45.4685 25.2095) (end -45.5295 25.1485) (width 0.254) (layer B.Cu) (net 3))
 (segment (start -42.2275 25.2095) (end -45.4685 25.2095) (width 0.254) (layer B.Cu) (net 3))
 (segment (start -35.7505 18.8325) (end -35.7505 17.5745) (width 0.254) (layer B.Cu) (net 3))
 (segment (start -42.1275 25.2095) (end -35.7505 18.8325) (width 0.254) (layer B.Cu) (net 3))
 (segment (start -42.2275 25.2095) (end -42.1275 25.2095) (width 0.254) (layer B.Cu) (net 3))
 (segment (start -39.8885 27.0485) (end -40.0275 26.9095) (width 0.254) (layer B.Cu) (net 2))
 (segment (start -36.8935 27.0485) (end -39.8885 27.0485) (width 0.254) (layer B.Cu) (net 2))
 (via (at -35.179 26.035) (size 0.8) (drill 0.4) (layers F.Cu B.Cu) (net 2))
 (segment (start -36.1925 27.0485) (end -35.179 26.035) (width 0.254) (layer B.Cu) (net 2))
 (segment (start -36.8935 27.0485) (end -36.1925 27.0485) (width 0.254) (layer B.Cu) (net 2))
 (via (at -35.433 22.352) (size 0.8) (drill 0.4) (layers F.Cu B.Cu) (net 2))
 (segment (start -35.179 22.606) (end -35.433 22.352) (width 0.254) (layer F.Cu) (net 2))
 (segment (start -35.179 26.035) (end -35.179 22.606) (width 0.254) (layer F.Cu) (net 2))
 (segment (start -34.9505 21.8695) (end -34.9505 17.5745) (width 0.254) (layer B.Cu) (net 2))
 (segment (start -35.433 22.352) (end -34.9505 21.8695) (width 0.254) (layer B.Cu) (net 2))
 (segment (start -28.0695 11.8745) (end -30.0505 11.8745) (width 0.254) (layer B.Cu) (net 37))
 (segment (start -25.6565 9.4615) (end -28.0695 11.8745) (width 0.254) (layer B.Cu) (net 37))
 (segment (start -7.8645 -2.9125) (end -5.969 -1.017) (width 0.254) (layer B.Cu) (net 46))
 (segment (start -11.7875 -2.9125) (end -7.8645 -2.9125) (width 0.254) (layer B.Cu) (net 46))
 (segment (start -5.041999 -3.389999) (end -5.969 -4.317) (width 0.254) (layer B.Cu) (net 47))
 (segment (start -5.041999 6.387001) (end -5.041999 -3.389999) (width 0.254) (layer B.Cu) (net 47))
 (segment (start -3.556 7.873) (end -5.041999 6.387001) (width 0.254) (layer B.Cu) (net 47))
 (segment (start -10.4 17.525) (end -11.7875 16.1375) (width 0.254) (layer B.Cu) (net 45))
 (segment (start -5.969 17.525) (end -10.4 17.525) (width 0.254) (layer B.Cu) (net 45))
 (segment (start -4.064 12.32) (end -5.969 14.225) (width 0.254) (layer B.Cu) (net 48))
 (segment (start -3.429 12.32) (end -4.064 12.32) (width 0.254) (layer B.Cu) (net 48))
 (segment (start 6.310499 15.185499) (end 7.2625 16.1375) (width 0.254) (layer B.Cu) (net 43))
 (segment (start 1.565539 15.185499) (end 6.310499 15.185499) (width 0.254) (layer B.Cu) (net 43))
 (segment (start 1.131038 15.62) (end 1.565539 15.185499) (width 0.254) (layer B.Cu) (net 43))
 (segment (start -3.429 15.62) (end 1.131038 15.62) (width 0.254) (layer B.Cu) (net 43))
 (segment (start 7.2625 2.522434) (end 7.2625 -2.9125) (width 0.254) (layer B.Cu) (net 42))
 (segment (start 5.211934 4.573) (end 7.2625 2.522434) (width 0.254) (layer B.Cu) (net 42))
 (segment (start -3.556 4.573) (end 5.211934 4.573) (width 0.254) (layer B.Cu) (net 42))
 (segment (start -43.383 -0.08575) (end -45.24375 1.775) (width 0.381) (layer B.Cu) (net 5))
 (segment (start -43.383 -1.723) (end -43.383 -0.08575) (width 0.381) (layer B.Cu) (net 5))
 (segment (start -18.0975 18.0975) (end -18.0975 -0.9525) (width 0.254) (layer B.Cu) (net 44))
 (segment (start 0.9525 18.0975) (end 2.7305 18.0975) (width 0.254) (layer F.Cu) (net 41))
 (segment (start 0.9525 16.3195) (end 0.9525 -0.9525) (width 0.254) (layer F.Cu) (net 41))
 (segment (start 2.7305 18.0975) (end 0.9525 16.3195) (width 0.254) (layer F.Cu) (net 41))
 (segment (start -29.852501 9.276501) (end -30.0505 9.4745) (width 0.254) (layer B.Cu) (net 39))
 (segment (start -28.912519 9.276501) (end -29.852501 9.276501) (width 0.254) (layer B.Cu) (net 39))
 (segment (start -25.51599 5.879972) (end -28.912519 9.276501) (width 0.254) (layer B.Cu) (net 39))
 (segment (start -25.51599 1.59026) (end -25.51599 5.879972) (width 0.254) (layer B.Cu) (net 39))
 (segment (start -26.19375 0.9125) (end -25.51599 1.59026) (width 0.254) (layer B.Cu) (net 39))
 (segment (start -26.19375 -0.9125) (end -33.6785 -0.9125) (width 0.254) (layer B.Cu) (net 6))
 (segment (start -33.6785 -0.9125) (end -36.703 -3.937) (width 0.254) (layer B.Cu) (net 6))
 (segment (start -42.583 -2.886602) (end -42.583 -1.723) (width 0.254) (layer B.Cu) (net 6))
 (segment (start -41.532602 -3.937) (end -42.583 -2.886602) (width 0.254) (layer B.Cu) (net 6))
 (segment (start -36.703 -3.937) (end -41.532602 -3.937) (width 0.254) (layer B.Cu) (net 6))
 (segment (start -41.783 -2.886602) (end -41.783 -1.723) (width 0.254) (layer B.Cu) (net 7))
 (segment (start -41.494601 -3.175001) (end -41.783 -2.886602) (width 0.254) (layer B.Cu) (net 7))
 (segment (start -39.671399 -3.175001) (end -41.494601 -3.175001) (width 0.254) (layer B.Cu) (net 7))
 (segment (start -39.605999 -1.031456) (end -39.605999 -3.109601) (width 0.254) (layer B.Cu) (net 7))
 (segment (start -38.620533 -0.04599) (end -39.605999 -1.031456) (width 0.254) (layer B.Cu) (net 7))
 (segment (start -29.35499 -0.04599) (end -38.620533 -0.04599) (width 0.254) (layer B.Cu) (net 7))
 (segment (start -39.605999 -3.109601) (end -39.671399 -3.175001) (width 0.254) (layer B.Cu) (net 7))
 (segment (start -26.543 2.766) (end -29.35499 -0.04599) (width 0.254) (layer B.Cu) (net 7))
 (segment (start -26.543 3.2785) (end -26.543 2.766) (width 0.254) (layer B.Cu) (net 7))
 (segment (start -28.16525 27.559) (end -25.1375 24.53125) (width 0.254) (layer B.Cu) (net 31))
 (segment (start -31.0915 27.559) (end -28.16525 27.559) (width 0.254) (layer B.Cu) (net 31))
 (segment (start -32.5505 26.1) (end -32.5505 17.5745) (width 0.254) (layer B.Cu) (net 31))
 (segment (start -31.0915 27.559) (end -32.5505 26.1) (width 0.254) (layer B.Cu) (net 31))
 (segment (start -42.4545 7.8745) (end -41.4505 7.8745) (width 0.254) (layer B.Cu) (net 17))
 (segment (start -44.3865 9.8065) (end -42.4545 7.8745) (width 0.254) (layer B.Cu) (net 17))
 (segment (start -44.3865 11.089) (end -44.3865 9.8065) (width 0.254) (layer B.Cu) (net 17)))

